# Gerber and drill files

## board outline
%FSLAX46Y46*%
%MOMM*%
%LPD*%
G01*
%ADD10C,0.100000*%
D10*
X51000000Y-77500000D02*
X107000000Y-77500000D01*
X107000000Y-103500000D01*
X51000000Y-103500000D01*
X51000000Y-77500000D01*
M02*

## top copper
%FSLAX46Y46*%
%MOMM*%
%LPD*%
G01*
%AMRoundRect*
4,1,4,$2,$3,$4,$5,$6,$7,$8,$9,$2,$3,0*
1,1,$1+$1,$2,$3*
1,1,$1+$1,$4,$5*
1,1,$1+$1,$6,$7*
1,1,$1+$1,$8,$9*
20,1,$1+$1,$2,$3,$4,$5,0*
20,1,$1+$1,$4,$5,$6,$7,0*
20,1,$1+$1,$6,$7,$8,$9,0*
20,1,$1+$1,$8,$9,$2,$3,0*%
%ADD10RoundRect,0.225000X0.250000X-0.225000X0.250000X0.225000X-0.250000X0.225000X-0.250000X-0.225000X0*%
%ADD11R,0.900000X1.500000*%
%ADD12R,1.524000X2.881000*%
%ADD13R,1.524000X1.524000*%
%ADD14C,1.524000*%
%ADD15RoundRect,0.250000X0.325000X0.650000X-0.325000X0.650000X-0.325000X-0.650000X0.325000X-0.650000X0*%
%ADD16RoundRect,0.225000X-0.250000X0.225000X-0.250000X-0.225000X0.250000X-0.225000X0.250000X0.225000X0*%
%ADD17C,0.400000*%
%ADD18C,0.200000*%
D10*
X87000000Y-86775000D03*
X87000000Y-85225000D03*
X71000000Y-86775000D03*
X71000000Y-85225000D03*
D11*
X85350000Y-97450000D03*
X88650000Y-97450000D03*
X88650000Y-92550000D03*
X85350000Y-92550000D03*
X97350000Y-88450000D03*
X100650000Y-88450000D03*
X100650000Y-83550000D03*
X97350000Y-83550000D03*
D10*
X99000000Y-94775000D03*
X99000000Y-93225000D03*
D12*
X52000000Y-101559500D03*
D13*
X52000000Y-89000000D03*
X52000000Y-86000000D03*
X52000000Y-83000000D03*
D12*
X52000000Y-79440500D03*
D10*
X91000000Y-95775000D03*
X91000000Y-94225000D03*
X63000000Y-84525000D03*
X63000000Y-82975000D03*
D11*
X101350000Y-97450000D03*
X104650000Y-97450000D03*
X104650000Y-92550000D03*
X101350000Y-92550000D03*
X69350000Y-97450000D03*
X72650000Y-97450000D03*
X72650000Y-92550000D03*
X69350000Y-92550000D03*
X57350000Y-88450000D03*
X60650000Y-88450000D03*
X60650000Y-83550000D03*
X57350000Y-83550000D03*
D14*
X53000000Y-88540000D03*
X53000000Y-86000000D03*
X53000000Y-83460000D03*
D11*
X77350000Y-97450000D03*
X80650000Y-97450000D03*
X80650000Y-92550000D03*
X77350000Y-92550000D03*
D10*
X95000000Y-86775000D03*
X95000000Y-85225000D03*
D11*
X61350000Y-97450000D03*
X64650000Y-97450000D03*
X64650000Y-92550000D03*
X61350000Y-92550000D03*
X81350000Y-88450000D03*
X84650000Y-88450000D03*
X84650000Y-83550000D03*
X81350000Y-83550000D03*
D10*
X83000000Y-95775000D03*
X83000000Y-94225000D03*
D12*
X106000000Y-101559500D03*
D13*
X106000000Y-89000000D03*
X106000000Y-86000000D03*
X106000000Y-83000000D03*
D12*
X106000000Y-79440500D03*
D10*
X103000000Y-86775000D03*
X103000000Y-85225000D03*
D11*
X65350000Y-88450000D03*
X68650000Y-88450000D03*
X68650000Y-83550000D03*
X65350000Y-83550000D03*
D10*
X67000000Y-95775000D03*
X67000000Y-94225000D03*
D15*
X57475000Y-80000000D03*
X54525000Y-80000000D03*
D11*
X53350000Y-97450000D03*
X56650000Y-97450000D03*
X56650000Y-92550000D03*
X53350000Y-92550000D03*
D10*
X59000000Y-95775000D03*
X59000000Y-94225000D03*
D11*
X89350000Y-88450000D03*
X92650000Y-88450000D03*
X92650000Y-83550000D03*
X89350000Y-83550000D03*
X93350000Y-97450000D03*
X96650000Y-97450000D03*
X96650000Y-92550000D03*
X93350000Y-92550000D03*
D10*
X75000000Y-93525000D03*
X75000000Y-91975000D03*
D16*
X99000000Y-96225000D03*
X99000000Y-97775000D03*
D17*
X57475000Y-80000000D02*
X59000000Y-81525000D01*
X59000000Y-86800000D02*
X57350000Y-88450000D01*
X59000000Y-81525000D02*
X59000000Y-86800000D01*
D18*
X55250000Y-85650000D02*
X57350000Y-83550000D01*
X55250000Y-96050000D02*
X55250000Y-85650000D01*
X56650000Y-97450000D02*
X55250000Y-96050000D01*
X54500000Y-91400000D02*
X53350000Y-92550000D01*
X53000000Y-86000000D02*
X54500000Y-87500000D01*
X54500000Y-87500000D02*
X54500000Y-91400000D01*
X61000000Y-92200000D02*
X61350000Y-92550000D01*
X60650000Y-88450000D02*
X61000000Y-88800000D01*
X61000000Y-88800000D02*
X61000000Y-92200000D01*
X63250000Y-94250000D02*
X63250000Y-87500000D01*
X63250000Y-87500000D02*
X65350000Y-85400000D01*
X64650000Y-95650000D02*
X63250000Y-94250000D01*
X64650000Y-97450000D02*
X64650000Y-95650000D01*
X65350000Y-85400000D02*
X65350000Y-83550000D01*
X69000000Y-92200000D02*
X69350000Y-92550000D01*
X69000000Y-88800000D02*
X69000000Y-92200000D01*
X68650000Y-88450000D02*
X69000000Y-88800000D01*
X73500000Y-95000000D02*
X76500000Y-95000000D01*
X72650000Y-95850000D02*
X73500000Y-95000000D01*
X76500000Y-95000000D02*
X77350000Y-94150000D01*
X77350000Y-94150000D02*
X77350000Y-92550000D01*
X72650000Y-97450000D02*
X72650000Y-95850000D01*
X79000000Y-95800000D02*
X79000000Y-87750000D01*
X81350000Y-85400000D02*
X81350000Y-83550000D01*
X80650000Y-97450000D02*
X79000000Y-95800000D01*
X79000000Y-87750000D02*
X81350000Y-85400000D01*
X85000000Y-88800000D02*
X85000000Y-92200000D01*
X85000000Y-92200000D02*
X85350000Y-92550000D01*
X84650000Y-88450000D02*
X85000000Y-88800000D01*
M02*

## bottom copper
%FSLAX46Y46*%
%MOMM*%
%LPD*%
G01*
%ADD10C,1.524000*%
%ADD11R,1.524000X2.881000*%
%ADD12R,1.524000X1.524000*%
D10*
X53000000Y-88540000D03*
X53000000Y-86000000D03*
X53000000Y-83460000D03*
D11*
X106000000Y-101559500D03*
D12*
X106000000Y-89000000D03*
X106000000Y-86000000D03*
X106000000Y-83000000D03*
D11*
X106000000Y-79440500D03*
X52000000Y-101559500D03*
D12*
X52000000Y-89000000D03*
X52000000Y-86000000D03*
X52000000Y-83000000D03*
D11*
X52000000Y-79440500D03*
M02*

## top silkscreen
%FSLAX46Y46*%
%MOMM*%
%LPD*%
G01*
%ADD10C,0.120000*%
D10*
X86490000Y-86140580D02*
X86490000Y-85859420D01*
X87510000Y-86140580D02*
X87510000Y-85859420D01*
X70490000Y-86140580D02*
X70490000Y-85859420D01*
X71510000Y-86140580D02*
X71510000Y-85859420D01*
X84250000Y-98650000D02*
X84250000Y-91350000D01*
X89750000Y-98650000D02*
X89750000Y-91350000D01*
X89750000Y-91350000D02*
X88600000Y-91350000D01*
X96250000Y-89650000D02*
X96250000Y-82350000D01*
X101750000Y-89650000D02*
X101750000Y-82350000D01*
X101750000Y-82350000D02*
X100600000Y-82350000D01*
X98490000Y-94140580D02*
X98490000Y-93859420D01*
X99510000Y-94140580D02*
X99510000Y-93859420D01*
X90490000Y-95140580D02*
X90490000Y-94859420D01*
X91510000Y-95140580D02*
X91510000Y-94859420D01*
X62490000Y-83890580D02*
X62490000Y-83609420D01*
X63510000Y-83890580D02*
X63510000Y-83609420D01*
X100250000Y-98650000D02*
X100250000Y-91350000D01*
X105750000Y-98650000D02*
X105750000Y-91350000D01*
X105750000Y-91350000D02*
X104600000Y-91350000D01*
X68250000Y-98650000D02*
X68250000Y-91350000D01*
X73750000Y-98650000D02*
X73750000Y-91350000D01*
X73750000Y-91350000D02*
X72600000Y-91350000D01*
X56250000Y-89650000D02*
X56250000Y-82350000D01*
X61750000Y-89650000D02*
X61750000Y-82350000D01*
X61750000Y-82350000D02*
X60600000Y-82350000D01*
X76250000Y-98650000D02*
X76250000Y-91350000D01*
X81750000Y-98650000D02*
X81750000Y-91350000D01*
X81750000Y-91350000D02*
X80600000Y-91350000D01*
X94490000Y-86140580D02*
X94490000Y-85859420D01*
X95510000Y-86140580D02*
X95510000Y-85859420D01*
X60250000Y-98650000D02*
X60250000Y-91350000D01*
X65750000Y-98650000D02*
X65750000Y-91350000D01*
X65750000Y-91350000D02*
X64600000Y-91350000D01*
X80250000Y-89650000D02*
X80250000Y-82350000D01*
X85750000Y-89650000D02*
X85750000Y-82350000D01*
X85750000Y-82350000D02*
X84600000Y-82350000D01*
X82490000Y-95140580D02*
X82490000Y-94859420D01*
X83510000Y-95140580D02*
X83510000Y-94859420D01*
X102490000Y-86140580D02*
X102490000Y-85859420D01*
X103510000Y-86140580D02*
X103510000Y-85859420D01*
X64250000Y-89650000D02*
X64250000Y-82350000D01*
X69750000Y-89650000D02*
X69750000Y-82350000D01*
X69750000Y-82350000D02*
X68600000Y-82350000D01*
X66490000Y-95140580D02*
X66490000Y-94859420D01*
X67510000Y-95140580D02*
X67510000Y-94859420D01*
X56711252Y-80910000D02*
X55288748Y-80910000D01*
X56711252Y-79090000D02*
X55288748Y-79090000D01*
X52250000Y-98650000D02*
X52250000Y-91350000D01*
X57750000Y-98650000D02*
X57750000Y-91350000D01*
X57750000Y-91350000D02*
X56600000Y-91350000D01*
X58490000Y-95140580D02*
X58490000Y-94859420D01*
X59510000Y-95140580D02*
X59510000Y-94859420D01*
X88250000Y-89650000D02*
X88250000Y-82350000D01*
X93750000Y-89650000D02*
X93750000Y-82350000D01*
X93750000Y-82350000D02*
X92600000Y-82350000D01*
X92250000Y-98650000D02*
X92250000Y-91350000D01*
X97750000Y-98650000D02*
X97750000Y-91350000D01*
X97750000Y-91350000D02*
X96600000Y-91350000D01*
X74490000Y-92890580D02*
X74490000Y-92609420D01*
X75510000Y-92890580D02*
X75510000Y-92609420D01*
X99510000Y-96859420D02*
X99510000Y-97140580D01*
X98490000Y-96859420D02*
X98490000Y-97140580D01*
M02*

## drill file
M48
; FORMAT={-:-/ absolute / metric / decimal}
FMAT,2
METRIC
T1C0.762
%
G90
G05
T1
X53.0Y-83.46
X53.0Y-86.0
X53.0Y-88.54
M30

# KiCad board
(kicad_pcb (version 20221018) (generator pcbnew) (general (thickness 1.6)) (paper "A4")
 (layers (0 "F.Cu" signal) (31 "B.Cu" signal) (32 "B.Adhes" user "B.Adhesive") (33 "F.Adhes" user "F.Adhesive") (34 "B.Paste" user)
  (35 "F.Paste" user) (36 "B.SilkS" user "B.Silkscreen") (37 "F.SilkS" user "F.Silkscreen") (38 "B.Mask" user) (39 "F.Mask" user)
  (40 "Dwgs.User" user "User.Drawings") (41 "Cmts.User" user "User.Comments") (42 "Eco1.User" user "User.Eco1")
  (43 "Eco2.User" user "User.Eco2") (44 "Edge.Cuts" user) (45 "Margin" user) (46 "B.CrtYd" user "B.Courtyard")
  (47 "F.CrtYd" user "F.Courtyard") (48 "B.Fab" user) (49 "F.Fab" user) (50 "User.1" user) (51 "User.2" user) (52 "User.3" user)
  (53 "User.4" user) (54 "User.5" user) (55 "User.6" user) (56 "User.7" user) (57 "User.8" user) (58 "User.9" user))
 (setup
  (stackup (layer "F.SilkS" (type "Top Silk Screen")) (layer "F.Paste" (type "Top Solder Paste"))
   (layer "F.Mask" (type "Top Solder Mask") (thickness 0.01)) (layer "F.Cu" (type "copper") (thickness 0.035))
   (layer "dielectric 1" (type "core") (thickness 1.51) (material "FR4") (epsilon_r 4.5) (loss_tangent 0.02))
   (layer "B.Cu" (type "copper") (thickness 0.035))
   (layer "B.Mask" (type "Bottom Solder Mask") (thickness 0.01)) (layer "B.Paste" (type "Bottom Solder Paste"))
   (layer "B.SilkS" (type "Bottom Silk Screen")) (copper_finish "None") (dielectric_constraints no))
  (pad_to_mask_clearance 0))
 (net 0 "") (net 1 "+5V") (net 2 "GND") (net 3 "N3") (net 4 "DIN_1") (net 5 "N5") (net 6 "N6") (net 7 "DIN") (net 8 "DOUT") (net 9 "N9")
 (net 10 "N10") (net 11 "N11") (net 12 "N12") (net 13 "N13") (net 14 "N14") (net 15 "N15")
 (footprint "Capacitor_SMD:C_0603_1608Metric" (layer "F.Cu") (at 87 86 90)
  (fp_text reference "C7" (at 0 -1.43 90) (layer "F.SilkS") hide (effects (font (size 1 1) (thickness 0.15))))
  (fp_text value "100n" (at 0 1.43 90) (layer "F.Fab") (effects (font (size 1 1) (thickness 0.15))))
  (fp_line (start -0.14058 -0.51) (end 0.14058 -0.51) (stroke (width 0.12) (type solid)) (layer "F.SilkS"))
  (fp_line (start -0.14058 0.51) (end 0.14058 0.51) (stroke (width 0.12) (type solid)) (layer "F.SilkS"))
  (pad "1" smd roundrect (at -0.775 0 90) (size 0.9 0.95) (layers "F.Cu" "F.Paste" "F.Mask") (roundrect_rratio 0.25) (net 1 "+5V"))
  (pad "2" smd roundrect (at 0.775 0 90) (size 0.9 0.95) (layers "F.Cu" "F.Paste" "F.Mask") (roundrect_rratio 0.25) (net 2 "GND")))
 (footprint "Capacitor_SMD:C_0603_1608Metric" (layer "F.Cu") (at 71 86 90)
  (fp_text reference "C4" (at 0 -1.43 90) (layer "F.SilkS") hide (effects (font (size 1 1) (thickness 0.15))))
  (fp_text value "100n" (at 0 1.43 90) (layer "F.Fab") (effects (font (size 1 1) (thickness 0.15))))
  (fp_line (start -0.14058 -0.51) (end 0.14058 -0.51) (stroke (width 0.12) (type solid)) (layer "F.SilkS"))
  (fp_line (start -0.14058 0.51) (end 0.14058 0.51) (stroke (width 0.12) (type solid)) (layer "F.SilkS"))
  (pad "1" smd roundrect (at -0.775 0 90) (size 0.9 0.95) (layers "F.Cu" "F.Paste" "F.Mask") (roundrect_rratio 0.25) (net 1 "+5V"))
  (pad "2" smd roundrect (at 0.775 0 90) (size 0.9 0.95) (layers "F.Cu" "F.Paste" "F.Mask") (roundrect_rratio 0.25) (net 2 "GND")))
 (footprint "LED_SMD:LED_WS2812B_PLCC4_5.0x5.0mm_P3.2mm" (layer "F.Cu") (at 87 95 90)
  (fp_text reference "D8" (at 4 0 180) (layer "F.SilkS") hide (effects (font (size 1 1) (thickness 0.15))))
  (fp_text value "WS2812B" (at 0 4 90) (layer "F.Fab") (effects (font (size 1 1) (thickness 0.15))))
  (fp_line (start -3.65 -2.75) (end 3.65 -2.75) (stroke (width 0.12) (type solid)) (layer "F.SilkS"))
  (fp_line (start -3.65 2.75) (end 3.65 2.75) (stroke (width 0.12) (type solid)) (layer "F.SilkS"))
  (fp_line (start 3.65 2.75) (end 3.65 1.6) (stroke (width 0.12) (type solid)) (layer "F.SilkS"))
  (pad "1" smd rect (at -2.45 -1.65 90) (size 1.5 0.9) (layers "F.Cu" "F.Paste" "F.Mask") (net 1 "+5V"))
  (pad "2" smd rect (at -2.45 1.65 90) (size 1.5 0.9) (layers "F.Cu" "F.Paste" "F.Mask") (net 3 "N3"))
  (pad "3" smd rect (at 2.45 1.65 90) (size 1.5 0.9) (layers "F.Cu" "F.Paste" "F.Mask") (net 2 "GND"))
  (pad "4" smd rect (at 2.45 -1.65 90) (size 1.5 0.9) (layers "F.Cu" "F.Paste" "F.Mask") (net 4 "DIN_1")))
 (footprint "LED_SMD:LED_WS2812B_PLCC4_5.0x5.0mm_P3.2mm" (layer "F.Cu") (at 99 86 90)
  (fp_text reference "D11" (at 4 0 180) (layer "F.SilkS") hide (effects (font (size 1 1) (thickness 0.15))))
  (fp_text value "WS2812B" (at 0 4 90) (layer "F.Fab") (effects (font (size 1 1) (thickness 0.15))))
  (fp_line (start -3.65 -2.75) (end 3.65 -2.75) (stroke (width 0.12) (type solid)) (layer "F.SilkS"))
  (fp_line (start -3.65 2.75) (end 3.65 2.75) (stroke (width 0.12) (type solid)) (layer "F.SilkS"))
  (fp_line (start 3.65 2.75) (end 3.65 1.6) (stroke (width 0.12) (type solid)) (layer "F.SilkS"))
  (pad "1" smd rect (at -2.45 -1.65 90) (size 1.5 0.9) (layers "F.Cu" "F.Paste" "F.Mask") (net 1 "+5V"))
  (pad "2" smd rect (at -2.45 1.65 90) (size 1.5 0.9) (layers "F.Cu" "F.Paste" "F.Mask") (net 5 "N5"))
  (pad "3" smd rect (at 2.45 1.65 90) (size 1.5 0.9) (layers "F.Cu" "F.Paste" "F.Mask") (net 2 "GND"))
  (pad "4" smd rect (at 2.45 -1.65 90) (size 1.5 0.9) (layers "F.Cu" "F.Paste" "F.Mask") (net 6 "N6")))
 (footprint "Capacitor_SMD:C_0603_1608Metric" (layer "F.Cu") (at 99 94 90)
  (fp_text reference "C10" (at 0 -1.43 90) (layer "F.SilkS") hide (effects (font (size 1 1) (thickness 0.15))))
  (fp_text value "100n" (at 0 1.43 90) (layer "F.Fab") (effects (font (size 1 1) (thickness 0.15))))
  (fp_line (start -0.14058 -0.51) (end 0.14058 -0.51) (stroke (width 0.12) (type solid)) (layer "F.SilkS"))
  (fp_line (start -0.14058 0.51) (end 0.14058 0.51) (stroke (width 0.12) (type solid)) (layer "F.SilkS"))
  (pad "1" smd roundrect (at -0.775 0 90) (size 0.9 0.95) (layers "F.Cu" "F.Paste" "F.Mask") (roundrect_rratio 0.25) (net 1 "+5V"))
  (pad "2" smd roundrect (at 0.775 0 90) (size 0.9 0.95) (layers "F.Cu" "F.Paste" "F.Mask") (roundrect_rratio 0.25) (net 2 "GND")))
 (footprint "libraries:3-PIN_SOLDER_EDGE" (layer "F.Cu") (at 52 100 90)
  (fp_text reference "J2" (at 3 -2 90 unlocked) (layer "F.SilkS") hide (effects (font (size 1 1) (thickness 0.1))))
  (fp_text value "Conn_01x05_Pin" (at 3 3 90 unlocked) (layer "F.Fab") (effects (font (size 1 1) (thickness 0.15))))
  (pad "1" connect rect (at -1.5595 0 90) (size 2.881 1.524) (layers "F.Cu" "F.Mask") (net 2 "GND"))
  (pad "2" connect rect (at 11 0 90) (size 1.524 1.524) (layers "F.Cu" "F.Mask") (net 1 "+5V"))
  (pad "3" connect rect (at 14 0 90) (size 1.524 1.524) (layers "F.Cu" "F.Mask") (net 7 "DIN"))
  (pad "4" connect rect (at 17 0 90) (size 1.524 1.524) (layers "F.Cu" "F.Mask") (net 2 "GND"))
  (pad "5" connect rect (at 20.5595 0 90) (size 2.881 1.524) (layers "F.Cu" "F.Mask") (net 2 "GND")))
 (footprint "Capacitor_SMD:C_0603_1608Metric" (layer "F.Cu") (at 91 95 90)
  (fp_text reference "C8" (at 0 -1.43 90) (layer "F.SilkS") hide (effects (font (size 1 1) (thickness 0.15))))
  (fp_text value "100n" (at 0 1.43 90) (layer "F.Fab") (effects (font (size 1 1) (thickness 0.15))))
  (fp_line (start -0.14058 -0.51) (end 0.14058 -0.51) (stroke (width 0.12) (type solid)) (layer "F.SilkS"))
  (fp_line (start -0.14058 0.51) (end 0.14058 0.51) (stroke (width 0.12) (type solid)) (layer "F.SilkS"))
  (pad "1" smd roundrect (at -0.775 0 90) (size 0.9 0.95) (layers "F.Cu" "F.Paste" "F.Mask") (roundrect_rratio 0.25) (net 1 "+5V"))
  (pad "2" smd roundrect (at 0.775 0 90) (size 0.9 0.95) (layers "F.Cu" "F.Paste" "F.Mask") (roundrect_rratio 0.25) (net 2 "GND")))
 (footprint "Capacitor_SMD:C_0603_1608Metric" (layer "F.Cu") (at 63 83.75 90)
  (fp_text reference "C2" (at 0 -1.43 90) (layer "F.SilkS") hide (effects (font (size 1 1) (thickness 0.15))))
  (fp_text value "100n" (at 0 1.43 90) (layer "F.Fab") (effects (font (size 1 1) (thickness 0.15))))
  (fp_line (start -0.14058 -0.51) (end 0.14058 -0.51) (stroke (width 0.12) (type solid)) (layer "F.SilkS"))
  (fp_line (start -0.14058 0.51) (end 0.14058 0.51) (stroke (width 0.12) (type solid)) (layer "F.SilkS"))
  (pad "1" smd roundrect (at -0.775 0 90) (size 0.9 0.95) (layers "F.Cu" "F.Paste" "F.Mask") (roundrect_rratio 0.25) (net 1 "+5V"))
  (pad "2" smd roundrect (at 0.775 0 90) (size 0.9 0.95) (layers "F.Cu" "F.Paste" "F.Mask") (roundrect_rratio 0.25) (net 2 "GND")))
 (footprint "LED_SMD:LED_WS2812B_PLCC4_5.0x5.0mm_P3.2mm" (layer "F.Cu") (at 103 95 90)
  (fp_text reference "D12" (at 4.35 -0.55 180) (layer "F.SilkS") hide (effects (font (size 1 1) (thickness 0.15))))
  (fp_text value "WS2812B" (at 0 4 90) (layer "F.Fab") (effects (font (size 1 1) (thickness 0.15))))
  (fp_line (start -3.65 -2.75) (end 3.65 -2.75) (stroke (width 0.12) (type solid)) (layer "F.SilkS"))
  (fp_line (start -3.65 2.75) (end 3.65 2.75) (stroke (width 0.12) (type solid)) (layer "F.SilkS"))
  (fp_line (start 3.65 2.75) (end 3.65 1.6) (stroke (width 0.12) (type solid)) (layer "F.SilkS"))
  (pad "1" smd rect (at -2.45 -1.65 90) (size 1.5 0.9) (layers "F.Cu" "F.Paste" "F.Mask") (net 1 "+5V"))
  (pad "2" smd rect (at -2.45 1.65 90) (size 1.5 0.9) (layers "F.Cu" "F.Paste" "F.Mask") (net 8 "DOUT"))
  (pad "3" smd rect (at 2.45 1.65 90) (size 1.5 0.9) (layers "F.Cu" "F.Paste" "F.Mask") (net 2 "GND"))
  (pad "4" smd rect (at 2.45 -1.65 90) (size 1.5 0.9) (layers "F.Cu" "F.Paste" "F.Mask") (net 5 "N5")))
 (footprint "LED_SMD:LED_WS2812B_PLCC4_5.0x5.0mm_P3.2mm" (layer "F.Cu") (at 71 95 90)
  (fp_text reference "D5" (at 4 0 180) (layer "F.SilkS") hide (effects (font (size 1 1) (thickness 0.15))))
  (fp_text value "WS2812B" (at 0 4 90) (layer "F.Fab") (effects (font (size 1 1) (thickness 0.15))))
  (fp_line (start -3.65 -2.75) (end 3.65 -2.75) (stroke (width 0.12) (type solid)) (layer "F.SilkS"))
  (fp_line (start -3.65 2.75) (end 3.65 2.75) (stroke (width 0.12) (type solid)) (layer "F.SilkS"))
  (fp_line (start 3.65 2.75) (end 3.65 1.6) (stroke (width 0.12) (type solid)) (layer "F.SilkS"))
  (pad "1" smd rect (at -2.45 -1.65 90) (size 1.5 0.9) (layers "F.Cu" "F.Paste" "F.Mask") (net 1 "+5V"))
  (pad "2" smd rect (at -2.45 1.65 90) (size 1.5 0.9) (layers "F.Cu" "F.Paste" "F.Mask") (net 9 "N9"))
  (pad "3" smd rect (at 2.45 1.65 90) (size 1.5 0.9) (layers "F.Cu" "F.Paste" "F.Mask") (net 2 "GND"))
  (pad "4" smd rect (at 2.45 -1.65 90) (size 1.5 0.9) (layers "F.Cu" "F.Paste" "F.Mask") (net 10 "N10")))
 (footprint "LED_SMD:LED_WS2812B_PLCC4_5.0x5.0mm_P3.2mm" (layer "F.Cu") (at 59 86 90)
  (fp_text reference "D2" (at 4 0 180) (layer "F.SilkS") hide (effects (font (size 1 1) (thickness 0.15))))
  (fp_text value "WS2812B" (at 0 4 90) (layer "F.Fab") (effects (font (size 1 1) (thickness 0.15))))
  (fp_line (start -3.65 -2.75) (end 3.65 -2.75) (stroke (width 0.12) (type solid)) (layer "F.SilkS"))
  (fp_line (start -3.65 2.75) (end 3.65 2.75) (stroke (width 0.12) (type solid)) (layer "F.SilkS"))
  (fp_line (start 3.65 2.75) (end 3.65 1.6) (stroke (width 0.12) (type solid)) (layer "F.SilkS"))
  (pad "1" smd rect (at -2.45 -1.65 90) (size 1.5 0.9) (layers "F.Cu" "F.Paste" "F.Mask") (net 1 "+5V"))
  (pad "2" smd rect (at -2.45 1.65 90) (size 1.5 0.9) (layers "F.Cu" "F.Paste" "F.Mask") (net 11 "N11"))
  (pad "3" smd rect (at 2.45 1.65 90) (size 1.5 0.9) (layers "F.Cu" "F.Paste" "F.Mask") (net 2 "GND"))
  (pad "4" smd rect (at 2.45 -1.65 90) (size 1.5 0.9) (layers "F.Cu" "F.Paste" "F.Mask") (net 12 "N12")))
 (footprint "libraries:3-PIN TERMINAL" (layer "F.Cu") (at 55.5 91 90)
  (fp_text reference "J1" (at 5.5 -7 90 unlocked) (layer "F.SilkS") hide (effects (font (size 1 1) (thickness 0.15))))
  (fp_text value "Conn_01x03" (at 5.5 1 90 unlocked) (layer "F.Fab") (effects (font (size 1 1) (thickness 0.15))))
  (pad "1" thru_hole circle (at 2.46 -2.5 90) (size 1.524 1.524) (drill 0.762) (layers "*.Cu" "*.Mask") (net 1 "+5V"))
  (pad "2" thru_hole circle (at 5 -2.5 90) (size 1.524 1.524) (drill 0.762) (layers "*.Cu" "*.Mask") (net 7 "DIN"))
  (pad "3" thru_hole circle (at 7.54 -2.5 90) (size 1.524 1.524) (drill 0.762) (layers "*.Cu" "*.Mask") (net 2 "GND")))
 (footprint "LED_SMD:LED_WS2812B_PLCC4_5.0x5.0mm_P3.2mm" (layer "F.Cu") (at 79 95 90)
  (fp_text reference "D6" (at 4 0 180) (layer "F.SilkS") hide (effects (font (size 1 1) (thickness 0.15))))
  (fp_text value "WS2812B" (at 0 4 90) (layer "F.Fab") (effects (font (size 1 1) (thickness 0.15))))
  (fp_line (start -3.65 -2.75) (end 3.65 -2.75) (stroke (width 0.12) (type solid)) (layer "F.SilkS"))
  (fp_line (start -3.65 2.75) (end 3.65 2.75) (stroke (width 0.12) (type solid)) (layer "F.SilkS"))
  (fp_line (start 3.65 2.75) (end 3.65 1.6) (stroke (width 0.12) (type solid)) (layer "F.SilkS"))
  (pad "1" smd rect (at -2.45 -1.65 90) (size 1.5 0.9) (layers "F.Cu" "F.Paste" "F.Mask") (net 1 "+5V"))
  (pad "2" smd rect (at -2.45 1.65 90) (size 1.5 0.9) (layers "F.Cu" "F.Paste" "F.Mask") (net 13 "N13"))
  (pad "3" smd rect (at 2.45 1.65 90) (size 1.5 0.9) (layers "F.Cu" "F.Paste" "F.Mask") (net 2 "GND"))
  (pad "4" smd rect (at 2.45 -1.65 90) (size 1.5 0.9) (layers "F.Cu" "F.Paste" "F.Mask") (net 9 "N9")))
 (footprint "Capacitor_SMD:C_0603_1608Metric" (layer "F.Cu") (at 95 86 90)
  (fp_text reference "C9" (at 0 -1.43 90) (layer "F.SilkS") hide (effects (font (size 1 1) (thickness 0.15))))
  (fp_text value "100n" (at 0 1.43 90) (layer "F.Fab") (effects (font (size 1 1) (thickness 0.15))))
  (fp_line (start -0.14058 -0.51) (end 0.14058 -0.51) (stroke (width 0.12) (type solid)) (layer "F.SilkS"))
  (fp_line (start -0.14058 0.51) (end 0.14058 0.51) (stroke (width 0.12) (type solid)) (layer "F.SilkS"))
  (pad "1" smd roundrect (at -0.775 0 90) (size 0.9 0.95) (layers "F.Cu" "F.Paste" "F.Mask") (roundrect_rratio 0.25) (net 1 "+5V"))
  (pad "2" smd roundrect (at 0.775 0 90) (size 0.9 0.95) (layers "F.Cu" "F.Paste" "F.Mask") (roundrect_rratio 0.25) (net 2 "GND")))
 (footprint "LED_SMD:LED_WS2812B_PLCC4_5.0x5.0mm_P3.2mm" (layer "F.Cu") (at 63 95 90)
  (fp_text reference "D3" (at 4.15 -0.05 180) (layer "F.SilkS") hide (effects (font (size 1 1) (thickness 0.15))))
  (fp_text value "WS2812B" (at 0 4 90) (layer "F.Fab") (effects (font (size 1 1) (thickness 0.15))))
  (fp_line (start -3.65 -2.75) (end 3.65 -2.75) (stroke (width 0.12) (type solid)) (layer "F.SilkS"))
  (fp_line (start -3.65 2.75) (end 3.65 2.75) (stroke (width 0.12) (type solid)) (layer "F.SilkS"))
  (fp_line (start 3.65 2.75) (end 3.65 1.6) (stroke (width 0.12) (type solid)) (layer "F.SilkS"))
  (pad "1" smd rect (at -2.45 -1.65 90) (size 1.5 0.9) (layers "F.Cu" "F.Paste" "F.Mask") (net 1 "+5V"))
  (pad "2" smd rect (at -2.45 1.65 90) (size 1.5 0.9) (layers "F.Cu" "F.Paste" "F.Mask") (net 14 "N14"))
  (pad "3" smd rect (at 2.45 1.65 90) (size 1.5 0.9) (layers "F.Cu" "F.Paste" "F.Mask") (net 2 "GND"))
  (pad "4" smd rect (at 2.45 -1.65 90) (size 1.5 0.9) (layers "F.Cu" "F.Paste" "F.Mask") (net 11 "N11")))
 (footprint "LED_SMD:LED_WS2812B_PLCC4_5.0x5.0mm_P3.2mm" (layer "F.Cu") (at 83 86 90)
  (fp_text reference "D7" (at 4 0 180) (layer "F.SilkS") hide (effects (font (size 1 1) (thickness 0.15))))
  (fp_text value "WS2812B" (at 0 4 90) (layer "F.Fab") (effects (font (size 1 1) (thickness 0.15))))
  (fp_line (start -3.65 -2.75) (end 3.65 -2.75) (stroke (width 0.12) (type solid)) (layer "F.SilkS"))
  (fp_line (start -3.65 2.75) (end 3.65 2.75) (stroke (width 0.12) (type solid)) (layer "F.SilkS"))
  (fp_line (start 3.65 2.75) (end 3.65 1.6) (stroke (width 0.12) (type solid)) (layer "F.SilkS"))
  (pad "1" smd rect (at -2.45 -1.65 90) (size 1.5 0.9) (layers "F.Cu" "F.Paste" "F.Mask") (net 1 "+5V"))
  (pad "2" smd rect (at -2.45 1.65 90) (size 1.5 0.9) (layers "F.Cu" "F.Paste" "F.Mask") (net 4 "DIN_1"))
  (pad "3" smd rect (at 2.45 1.65 90) (size 1.5 0.9) (layers "F.Cu" "F.Paste" "F.Mask") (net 2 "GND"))
  (pad "4" smd rect (at 2.45 -1.65 90) (size 1.5 0.9) (layers "F.Cu" "F.Paste" "F.Mask") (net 13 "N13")))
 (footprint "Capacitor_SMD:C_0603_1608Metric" (layer "F.Cu") (at 83 95 90)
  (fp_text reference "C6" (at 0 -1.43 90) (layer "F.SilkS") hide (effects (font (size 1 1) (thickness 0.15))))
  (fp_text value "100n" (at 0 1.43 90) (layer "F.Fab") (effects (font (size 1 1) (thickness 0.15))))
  (fp_line (start -0.14058 -0.51) (end 0.14058 -0.51) (stroke (width 0.12) (type solid)) (layer "F.SilkS"))
  (fp_line (start -0.14058 0.51) (end 0.14058 0.51) (stroke (width 0.12) (type solid)) (layer "F.SilkS"))
  (pad "1" smd roundrect (at -0.775 0 90) (size 0.9 0.95) (layers "F.Cu" "F.Paste" "F.Mask") (roundrect_rratio 0.25) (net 1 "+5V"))
  (pad "2" smd roundrect (at 0.775 0 90) (size 0.9 0.95) (layers "F.Cu" "F.Paste" "F.Mask") (roundrect_rratio 0.25) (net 2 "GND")))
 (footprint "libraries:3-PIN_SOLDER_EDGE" (layer "F.Cu") (at 106 100 90)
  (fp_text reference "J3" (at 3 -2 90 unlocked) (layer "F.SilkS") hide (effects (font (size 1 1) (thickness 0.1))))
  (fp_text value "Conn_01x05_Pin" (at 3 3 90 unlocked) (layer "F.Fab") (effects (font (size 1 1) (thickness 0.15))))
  (pad "1" connect rect (at -1.5595 0 90) (size 2.881 1.524) (layers "F.Cu" "F.Mask") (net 2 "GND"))
  (pad "2" connect rect (at 11 0 90) (size 1.524 1.524) (layers "F.Cu" "F.Mask") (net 1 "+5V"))
  (pad "3" connect rect (at 14 0 90) (size 1.524 1.524) (layers "F.Cu" "F.Mask") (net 8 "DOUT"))
  (pad "4" connect rect (at 17 0 90) (size 1.524 1.524) (layers "F.Cu" "F.Mask") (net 2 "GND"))
  (pad "5" connect rect (at 20.5595 0 90) (size 2.881 1.524) (layers "F.Cu" "F.Mask") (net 2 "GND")))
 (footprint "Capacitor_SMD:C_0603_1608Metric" (layer "F.Cu") (at 103 86 90)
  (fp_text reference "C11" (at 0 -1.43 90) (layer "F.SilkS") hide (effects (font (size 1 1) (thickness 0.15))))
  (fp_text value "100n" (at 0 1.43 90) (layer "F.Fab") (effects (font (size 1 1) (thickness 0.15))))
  (fp_line (start -0.14058 -0.51) (end 0.14058 -0.51) (stroke (width 0.12) (type solid)) (layer "F.SilkS"))
  (fp_line (start -0.14058 0.51) (end 0.14058 0.51) (stroke (width 0.12) (type solid)) (layer "F.SilkS"))
  (pad "1" smd roundrect (at -0.775 0 90) (size 0.9 0.95) (layers "F.Cu" "F.Paste" "F.Mask") (roundrect_rratio 0.25) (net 1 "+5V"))
  (pad "2" smd roundrect (at 0.775 0 90) (size 0.9 0.95) (layers "F.Cu" "F.Paste" "F.Mask") (roundrect_rratio 0.25) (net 2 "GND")))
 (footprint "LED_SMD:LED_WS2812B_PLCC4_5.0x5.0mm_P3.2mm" (layer "F.Cu") (at 67 86 90)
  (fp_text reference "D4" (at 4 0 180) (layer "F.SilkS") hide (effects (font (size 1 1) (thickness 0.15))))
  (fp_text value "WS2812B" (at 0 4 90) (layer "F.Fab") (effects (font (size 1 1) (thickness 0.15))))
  (fp_line (start -3.65 -2.75) (end 3.65 -2.75) (stroke (width 0.12) (type solid)) (layer "F.SilkS"))
  (fp_line (start -3.65 2.75) (end 3.65 2.75) (stroke (width 0.12) (type solid)) (layer "F.SilkS"))
  (fp_line (start 3.65 2.75) (end 3.65 1.6) (stroke (width 0.12) (type solid)) (layer "F.SilkS"))
  (pad "1" smd rect (at -2.45 -1.65 90) (size 1.5 0.9) (layers "F.Cu" "F.Paste" "F.Mask") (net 1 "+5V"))
  (pad "2" smd rect (at -2.45 1.65 90) (size 1.5 0.9) (layers "F.Cu" "F.Paste" "F.Mask") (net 10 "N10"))
  (pad "3" smd rect (at 2.45 1.65 90) (size 1.5 0.9) (layers "F.Cu" "F.Paste" "F.Mask") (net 2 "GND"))
  (pad "4" smd rect (at 2.45 -1.65 90) (size 1.5 0.9) (layers "F.Cu" "F.Paste" "F.Mask") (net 14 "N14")))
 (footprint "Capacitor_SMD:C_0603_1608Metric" (layer "F.Cu") (at 67 95 90)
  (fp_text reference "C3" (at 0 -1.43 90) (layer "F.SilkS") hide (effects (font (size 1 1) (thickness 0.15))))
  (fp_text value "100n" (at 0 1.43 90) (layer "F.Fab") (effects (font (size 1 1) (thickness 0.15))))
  (fp_line (start -0.14058 -0.51) (end 0.14058 -0.51) (stroke (width 0.12) (type solid)) (layer "F.SilkS"))
  (fp_line (start -0.14058 0.51) (end 0.14058 0.51) (stroke (width 0.12) (type solid)) (layer "F.SilkS"))
  (pad "1" smd roundrect (at -0.775 0 90) (size 0.9 0.95) (layers "F.Cu" "F.Paste" "F.Mask") (roundrect_rratio 0.25) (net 1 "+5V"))
  (pad "2" smd roundrect (at 0.775 0 90) (size 0.9 0.95) (layers "F.Cu" "F.Paste" "F.Mask") (roundrect_rratio 0.25) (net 2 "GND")))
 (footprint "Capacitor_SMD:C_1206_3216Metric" (layer "F.Cu") (at 56 80 180)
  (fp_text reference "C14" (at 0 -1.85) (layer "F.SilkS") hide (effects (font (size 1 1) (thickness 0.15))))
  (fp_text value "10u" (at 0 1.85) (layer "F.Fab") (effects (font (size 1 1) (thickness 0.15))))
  (fp_line (start -0.711252 -0.91) (end 0.711252 -0.91) (stroke (width 0.12) (type solid)) (layer "F.SilkS"))
  (fp_line (start -0.711252 0.91) (end 0.711252 0.91) (stroke (width 0.12) (type solid)) (layer "F.SilkS"))
  (pad "1" smd roundrect (at -1.475 0 180) (size 1.15 1.8) (layers "F.Cu" "F.Paste" "F.Mask") (roundrect_rratio 0.217391) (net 1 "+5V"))
  (pad "2" smd roundrect (at 1.475 0 180) (size 1.15 1.8) (layers "F.Cu" "F.Paste" "F.Mask") (roundrect_rratio 0.217391) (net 2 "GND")))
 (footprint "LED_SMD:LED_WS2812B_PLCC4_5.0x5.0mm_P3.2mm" (layer "F.Cu") (at 55 95 90)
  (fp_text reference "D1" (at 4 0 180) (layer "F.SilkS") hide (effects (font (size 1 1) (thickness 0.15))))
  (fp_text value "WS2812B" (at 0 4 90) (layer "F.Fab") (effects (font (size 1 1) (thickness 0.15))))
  (fp_line (start -3.65 -2.75) (end 3.65 -2.75) (stroke (width 0.12) (type solid)) (layer "F.SilkS"))
  (fp_line (start -3.65 2.75) (end 3.65 2.75) (stroke (width 0.12) (type solid)) (layer "F.SilkS"))
  (fp_line (start 3.65 2.75) (end 3.65 1.6) (stroke (width 0.12) (type solid)) (layer "F.SilkS"))
  (pad "1" smd rect (at -2.45 -1.65 90) (size 1.5 0.9) (layers "F.Cu" "F.Paste" "F.Mask") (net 1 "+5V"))
  (pad "2" smd rect (at -2.45 1.65 90) (size 1.5 0.9) (layers "F.Cu" "F.Paste" "F.Mask") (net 12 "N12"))
  (pad "3" smd rect (at 2.45 1.65 90) (size 1.5 0.9) (layers "F.Cu" "F.Paste" "F.Mask") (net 2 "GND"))
  (pad "4" smd rect (at 2.45 -1.65 90) (size 1.5 0.9) (layers "F.Cu" "F.Paste" "F.Mask") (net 7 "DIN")))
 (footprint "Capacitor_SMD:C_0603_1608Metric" (layer "F.Cu") (at 59 95 90)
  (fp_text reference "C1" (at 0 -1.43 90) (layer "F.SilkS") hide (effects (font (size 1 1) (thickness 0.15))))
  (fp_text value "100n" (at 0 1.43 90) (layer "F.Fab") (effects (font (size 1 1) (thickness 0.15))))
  (fp_line (start -0.14058 -0.51) (end 0.14058 -0.51) (stroke (width 0.12) (type solid)) (layer "F.SilkS"))
  (fp_line (start -0.14058 0.51) (end 0.14058 0.51) (stroke (width 0.12) (type solid)) (layer "F.SilkS"))
  (pad "1" smd roundrect (at -0.775 0 90) (size 0.9 0.95) (layers "F.Cu" "F.Paste" "F.Mask") (roundrect_rratio 0.25) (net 1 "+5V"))
  (pad "2" smd roundrect (at 0.775 0 90) (size 0.9 0.95) (layers "F.Cu" "F.Paste" "F.Mask") (roundrect_rratio 0.25) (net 2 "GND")))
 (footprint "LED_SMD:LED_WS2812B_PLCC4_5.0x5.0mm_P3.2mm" (layer "F.Cu") (at 91 86 90)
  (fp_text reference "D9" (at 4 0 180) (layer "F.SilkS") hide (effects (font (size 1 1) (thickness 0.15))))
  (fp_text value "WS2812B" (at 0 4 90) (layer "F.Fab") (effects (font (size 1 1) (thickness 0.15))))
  (fp_line (start -3.65 -2.75) (end 3.65 -2.75) (stroke (width 0.12) (type solid)) (layer "F.SilkS"))
  (fp_line (start -3.65 2.75) (end 3.65 2.75) (stroke (width 0.12) (type solid)) (layer "F.SilkS"))
  (fp_line (start 3.65 2.75) (end 3.65 1.6) (stroke (width 0.12) (type solid)) (layer "F.SilkS"))
  (pad "1" smd rect (at -2.45 -1.65 90) (size 1.5 0.9) (layers "F.Cu" "F.Paste" "F.Mask") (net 1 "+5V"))
  (pad "2" smd rect (at -2.45 1.65 90) (size 1.5 0.9) (layers "F.Cu" "F.Paste" "F.Mask") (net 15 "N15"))
  (pad "3" smd rect (at 2.45 1.65 90) (size 1.5 0.9) (layers "F.Cu" "F.Paste" "F.Mask") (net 2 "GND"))
  (pad "4" smd rect (at 2.45 -1.65 90) (size 1.5 0.9) (layers "F.Cu" "F.Paste" "F.Mask") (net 3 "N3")))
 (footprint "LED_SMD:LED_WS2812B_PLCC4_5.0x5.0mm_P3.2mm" (layer "F.Cu") (at 95 95 90)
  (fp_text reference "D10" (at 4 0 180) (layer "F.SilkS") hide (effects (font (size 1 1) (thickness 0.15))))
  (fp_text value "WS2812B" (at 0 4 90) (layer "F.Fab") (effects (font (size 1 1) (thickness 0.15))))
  (fp_line (start -3.65 -2.75) (end 3.65 -2.75) (stroke (width 0.12) (type solid)) (layer "F.SilkS"))
  (fp_line (start -3.65 2.75) (end 3.65 2.75) (stroke (width 0.12) (type solid)) (layer "F.SilkS"))
  (fp_line (start 3.65 2.75) (end 3.65 1.6) (stroke (width 0.12) (type solid)) (layer "F.SilkS"))
  (pad "1" smd rect (at -2.45 -1.65 90) (size 1.5 0.9) (layers "F.Cu" "F.Paste" "F.Mask") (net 1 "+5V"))
  (pad "2" smd rect (at -2.45 1.65 90) (size 1.5 0.9) (layers "F.Cu" "F.Paste" "F.Mask") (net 6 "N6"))
  (pad "3" smd rect (at 2.45 1.65 90) (size 1.5 0.9) (layers "F.Cu" "F.Paste" "F.Mask") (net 2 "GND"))
  (pad "4" smd rect (at 2.45 -1.65 90) (size 1.5 0.9) (layers "F.Cu" "F.Paste" "F.Mask") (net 15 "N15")))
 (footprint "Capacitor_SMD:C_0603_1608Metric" (layer "F.Cu") (at 75 92.75 90)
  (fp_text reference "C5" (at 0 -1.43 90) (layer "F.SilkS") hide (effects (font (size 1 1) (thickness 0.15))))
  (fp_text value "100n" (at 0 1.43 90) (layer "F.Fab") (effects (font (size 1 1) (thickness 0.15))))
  (fp_line (start -0.14058 -0.51) (end 0.14058 -0.51) (stroke (width 0.12) (type solid)) (layer "F.SilkS"))
  (fp_line (start -0.14058 0.51) (end 0.14058 0.51) (stroke (width 0.12) (type solid)) (layer "F.SilkS"))
  (pad "1" smd roundrect (at -0.775 0 90) (size 0.9 0.95) (layers "F.Cu" "F.Paste" "F.Mask") (roundrect_rratio 0.25) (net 1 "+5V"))
  (pad "2" smd roundrect (at 0.775 0 90) (size 0.9 0.95) (layers "F.Cu" "F.Paste" "F.Mask") (roundrect_rratio 0.25) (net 2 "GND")))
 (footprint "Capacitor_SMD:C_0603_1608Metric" (layer "F.Cu") (at 99 97 -90)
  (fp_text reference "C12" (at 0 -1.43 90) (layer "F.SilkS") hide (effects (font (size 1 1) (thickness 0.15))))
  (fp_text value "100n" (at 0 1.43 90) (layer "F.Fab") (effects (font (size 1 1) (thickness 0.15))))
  (fp_line (start -0.14058 -0.51) (end 0.14058 -0.51) (stroke (width 0.12) (type solid)) (layer "F.SilkS"))
  (fp_line (start -0.14058 0.51) (end 0.14058 0.51) (stroke (width 0.12) (type solid)) (layer "F.SilkS"))
  (pad "1" smd roundrect (at -0.775 0 270) (size 0.9 0.95) (layers "F.Cu" "F.Paste" "F.Mask") (roundrect_rratio 0.25) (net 1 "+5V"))
  (pad "2" smd roundrect (at 0.775 0 270) (size 0.9 0.95) (layers "F.Cu" "F.Paste" "F.Mask") (roundrect_rratio 0.25) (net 2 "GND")))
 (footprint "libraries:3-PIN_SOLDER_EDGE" (layer "B.Cu") (at 106 100 90)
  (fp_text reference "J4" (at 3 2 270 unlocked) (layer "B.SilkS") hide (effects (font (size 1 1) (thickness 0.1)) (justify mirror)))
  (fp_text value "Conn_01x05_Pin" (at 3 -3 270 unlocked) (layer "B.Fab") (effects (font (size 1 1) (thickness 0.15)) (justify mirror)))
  (pad "1" connect rect (at -1.5595 0 90) (size 2.881 1.524) (layers "B.Cu" "B.Mask") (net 2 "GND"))
  (pad "2" connect rect (at 11 0 90) (size 1.524 1.524) (layers "B.Cu" "B.Mask") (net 1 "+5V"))
  (pad "3" connect rect (at 14 0 90) (size 1.524 1.524) (layers "B.Cu" "B.Mask") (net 8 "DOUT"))
  (pad "4" connect rect (at 17 0 90) (size 1.524 1.524) (layers "B.Cu" "B.Mask") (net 2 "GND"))
  (pad "5" connect rect (at 20.5595 0 90) (size 2.881 1.524) (layers "B.Cu" "B.Mask") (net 2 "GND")))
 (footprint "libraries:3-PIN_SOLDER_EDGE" (layer "B.Cu") (at 52 100 90)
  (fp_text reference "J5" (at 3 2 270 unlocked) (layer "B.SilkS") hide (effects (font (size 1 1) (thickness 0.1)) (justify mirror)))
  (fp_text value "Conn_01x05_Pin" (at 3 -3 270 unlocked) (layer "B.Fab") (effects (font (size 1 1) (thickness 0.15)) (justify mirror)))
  (pad "1" connect rect (at -1.5595 0 90) (size 2.881 1.524) (layers "B.Cu" "B.Mask") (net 2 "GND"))
  (pad "2" connect rect (at 11 0 90) (size 1.524 1.524) (layers "B.Cu" "B.Mask") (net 1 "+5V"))
  (pad "3" connect rect (at 14 0 90) (size 1.524 1.524) (layers "B.Cu" "B.Mask") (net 7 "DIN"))
  (pad "4" connect rect (at 17 0 90) (size 1.524 1.524) (layers "B.Cu" "B.Mask") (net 2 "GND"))
  (pad "5" connect rect (at 20.5595 0 90) (size 2.881 1.524) (layers "B.Cu" "B.Mask") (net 2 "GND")))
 (gr_rect (start 51 77.5) (end 107 103.5) (stroke (width 0.1) (type default)) (fill none) (layer "Edge.Cuts"))
 (segment (start 57.475 80) (end 59 81.525) (width 0.4) (layer "F.Cu") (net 1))
 (segment (start 59 86.8) (end 57.35 88.45) (width 0.4) (layer "F.Cu") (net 1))
 (segment (start 59 81.525) (end 59 86.8) (width 0.4) (layer "F.Cu") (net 1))
 (segment (start 55.25 85.65) (end 57.35 83.55) (width 0.2) (layer "F.Cu") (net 12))
 (segment (start 55.25 96.05) (end 55.25 85.65) (width 0.2) (layer "F.Cu") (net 12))
 (segment (start 56.65 97.45) (end 55.25 96.05) (width 0.2) (layer "F.Cu") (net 12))
 (segment (start 54.5 91.4) (end 53.35 92.55) (width 0.2) (layer "F.Cu") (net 7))
 (segment (start 53 86) (end 54.5 87.5) (width 0.2) (layer "F.Cu") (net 7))
 (segment (start 54.5 87.5) (end 54.5 91.4) (width 0.2) (layer "F.Cu") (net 7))
 (segment (start 61 92.2) (end 61.35 92.55) (width 0.2) (layer "F.Cu") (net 11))
 (segment (start 60.65 88.45) (end 61 88.8) (width 0.2) (layer "F.Cu") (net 11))
 (segment (start 61 88.8) (end 61 92.2) (width 0.2) (layer "F.Cu") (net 11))
 (segment (start 63.25 94.25) (end 63.25 87.5) (width 0.2) (layer "F.Cu") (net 14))
 (segment (start 63.25 87.5) (end 65.35 85.4) (width 0.2) (layer "F.Cu") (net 14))
 (segment (start 64.65 95.65) (end 63.25 94.25) (width 0.2) (layer "F.Cu") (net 14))
 (segment (start 64.65 97.45) (end 64.65 95.65) (width 0.2) (layer "F.Cu") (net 14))
 (segment (start 65.35 85.4) (end 65.35 83.55) (width 0.2) (layer "F.Cu") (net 14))
 (segment (start 69 92.2) (end 69.35 92.55) (width 0.2) (layer "F.Cu") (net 10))
 (segment (start 69 88.8) (end 69 92.2) (width 0.2) (layer "F.Cu") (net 10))
 (segment (start 68.65 88.45) (end 69 88.8) (width 0.2) (layer "F.Cu") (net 10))
 (segment (start 73.5 95) (end 76.5 95) (width 0.2) (layer "F.Cu") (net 9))
 (segment (start 72.65 95.85) (end 73.5 95) (width 0.2) (layer "F.Cu") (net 9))
 (segment (start 76.5 95) (end 77.35 94.15) (width 0.2) (layer "F.Cu") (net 9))
 (segment (start 77.35 94.15) (end 77.35 92.55) (width 0.2) (layer "F.Cu") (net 9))
 (segment (start 72.65 97.45) (end 72.65 95.85) (width 0.2) (layer "F.Cu") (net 9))
 (segment (start 79 95.8) (end 79 87.75) (width 0.2) (layer "F.Cu") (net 13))
 (segment (start 81.35 85.4) (end 81.35 83.55) (width 0.2) (layer "F.Cu") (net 13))
 (segment (start 80.65 97.45) (end 79 95.8) (width 0.2) (layer "F.Cu") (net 13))
 (segment (start 79 87.75) (end 81.35 85.4) (width 0.2) (layer "F.Cu") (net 13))
 (segment (start 85 88.8) (end 85 92.2) (width 0.2) (layer "F.Cu") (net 4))
 (segment (start 85 92.2) (end 85.35 92.55) (width 0.2) (layer "F.Cu") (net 4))
 (segment (start 84.65 88.45) (end 85 88.8) (width 0.2) (layer "F.Cu") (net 4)))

